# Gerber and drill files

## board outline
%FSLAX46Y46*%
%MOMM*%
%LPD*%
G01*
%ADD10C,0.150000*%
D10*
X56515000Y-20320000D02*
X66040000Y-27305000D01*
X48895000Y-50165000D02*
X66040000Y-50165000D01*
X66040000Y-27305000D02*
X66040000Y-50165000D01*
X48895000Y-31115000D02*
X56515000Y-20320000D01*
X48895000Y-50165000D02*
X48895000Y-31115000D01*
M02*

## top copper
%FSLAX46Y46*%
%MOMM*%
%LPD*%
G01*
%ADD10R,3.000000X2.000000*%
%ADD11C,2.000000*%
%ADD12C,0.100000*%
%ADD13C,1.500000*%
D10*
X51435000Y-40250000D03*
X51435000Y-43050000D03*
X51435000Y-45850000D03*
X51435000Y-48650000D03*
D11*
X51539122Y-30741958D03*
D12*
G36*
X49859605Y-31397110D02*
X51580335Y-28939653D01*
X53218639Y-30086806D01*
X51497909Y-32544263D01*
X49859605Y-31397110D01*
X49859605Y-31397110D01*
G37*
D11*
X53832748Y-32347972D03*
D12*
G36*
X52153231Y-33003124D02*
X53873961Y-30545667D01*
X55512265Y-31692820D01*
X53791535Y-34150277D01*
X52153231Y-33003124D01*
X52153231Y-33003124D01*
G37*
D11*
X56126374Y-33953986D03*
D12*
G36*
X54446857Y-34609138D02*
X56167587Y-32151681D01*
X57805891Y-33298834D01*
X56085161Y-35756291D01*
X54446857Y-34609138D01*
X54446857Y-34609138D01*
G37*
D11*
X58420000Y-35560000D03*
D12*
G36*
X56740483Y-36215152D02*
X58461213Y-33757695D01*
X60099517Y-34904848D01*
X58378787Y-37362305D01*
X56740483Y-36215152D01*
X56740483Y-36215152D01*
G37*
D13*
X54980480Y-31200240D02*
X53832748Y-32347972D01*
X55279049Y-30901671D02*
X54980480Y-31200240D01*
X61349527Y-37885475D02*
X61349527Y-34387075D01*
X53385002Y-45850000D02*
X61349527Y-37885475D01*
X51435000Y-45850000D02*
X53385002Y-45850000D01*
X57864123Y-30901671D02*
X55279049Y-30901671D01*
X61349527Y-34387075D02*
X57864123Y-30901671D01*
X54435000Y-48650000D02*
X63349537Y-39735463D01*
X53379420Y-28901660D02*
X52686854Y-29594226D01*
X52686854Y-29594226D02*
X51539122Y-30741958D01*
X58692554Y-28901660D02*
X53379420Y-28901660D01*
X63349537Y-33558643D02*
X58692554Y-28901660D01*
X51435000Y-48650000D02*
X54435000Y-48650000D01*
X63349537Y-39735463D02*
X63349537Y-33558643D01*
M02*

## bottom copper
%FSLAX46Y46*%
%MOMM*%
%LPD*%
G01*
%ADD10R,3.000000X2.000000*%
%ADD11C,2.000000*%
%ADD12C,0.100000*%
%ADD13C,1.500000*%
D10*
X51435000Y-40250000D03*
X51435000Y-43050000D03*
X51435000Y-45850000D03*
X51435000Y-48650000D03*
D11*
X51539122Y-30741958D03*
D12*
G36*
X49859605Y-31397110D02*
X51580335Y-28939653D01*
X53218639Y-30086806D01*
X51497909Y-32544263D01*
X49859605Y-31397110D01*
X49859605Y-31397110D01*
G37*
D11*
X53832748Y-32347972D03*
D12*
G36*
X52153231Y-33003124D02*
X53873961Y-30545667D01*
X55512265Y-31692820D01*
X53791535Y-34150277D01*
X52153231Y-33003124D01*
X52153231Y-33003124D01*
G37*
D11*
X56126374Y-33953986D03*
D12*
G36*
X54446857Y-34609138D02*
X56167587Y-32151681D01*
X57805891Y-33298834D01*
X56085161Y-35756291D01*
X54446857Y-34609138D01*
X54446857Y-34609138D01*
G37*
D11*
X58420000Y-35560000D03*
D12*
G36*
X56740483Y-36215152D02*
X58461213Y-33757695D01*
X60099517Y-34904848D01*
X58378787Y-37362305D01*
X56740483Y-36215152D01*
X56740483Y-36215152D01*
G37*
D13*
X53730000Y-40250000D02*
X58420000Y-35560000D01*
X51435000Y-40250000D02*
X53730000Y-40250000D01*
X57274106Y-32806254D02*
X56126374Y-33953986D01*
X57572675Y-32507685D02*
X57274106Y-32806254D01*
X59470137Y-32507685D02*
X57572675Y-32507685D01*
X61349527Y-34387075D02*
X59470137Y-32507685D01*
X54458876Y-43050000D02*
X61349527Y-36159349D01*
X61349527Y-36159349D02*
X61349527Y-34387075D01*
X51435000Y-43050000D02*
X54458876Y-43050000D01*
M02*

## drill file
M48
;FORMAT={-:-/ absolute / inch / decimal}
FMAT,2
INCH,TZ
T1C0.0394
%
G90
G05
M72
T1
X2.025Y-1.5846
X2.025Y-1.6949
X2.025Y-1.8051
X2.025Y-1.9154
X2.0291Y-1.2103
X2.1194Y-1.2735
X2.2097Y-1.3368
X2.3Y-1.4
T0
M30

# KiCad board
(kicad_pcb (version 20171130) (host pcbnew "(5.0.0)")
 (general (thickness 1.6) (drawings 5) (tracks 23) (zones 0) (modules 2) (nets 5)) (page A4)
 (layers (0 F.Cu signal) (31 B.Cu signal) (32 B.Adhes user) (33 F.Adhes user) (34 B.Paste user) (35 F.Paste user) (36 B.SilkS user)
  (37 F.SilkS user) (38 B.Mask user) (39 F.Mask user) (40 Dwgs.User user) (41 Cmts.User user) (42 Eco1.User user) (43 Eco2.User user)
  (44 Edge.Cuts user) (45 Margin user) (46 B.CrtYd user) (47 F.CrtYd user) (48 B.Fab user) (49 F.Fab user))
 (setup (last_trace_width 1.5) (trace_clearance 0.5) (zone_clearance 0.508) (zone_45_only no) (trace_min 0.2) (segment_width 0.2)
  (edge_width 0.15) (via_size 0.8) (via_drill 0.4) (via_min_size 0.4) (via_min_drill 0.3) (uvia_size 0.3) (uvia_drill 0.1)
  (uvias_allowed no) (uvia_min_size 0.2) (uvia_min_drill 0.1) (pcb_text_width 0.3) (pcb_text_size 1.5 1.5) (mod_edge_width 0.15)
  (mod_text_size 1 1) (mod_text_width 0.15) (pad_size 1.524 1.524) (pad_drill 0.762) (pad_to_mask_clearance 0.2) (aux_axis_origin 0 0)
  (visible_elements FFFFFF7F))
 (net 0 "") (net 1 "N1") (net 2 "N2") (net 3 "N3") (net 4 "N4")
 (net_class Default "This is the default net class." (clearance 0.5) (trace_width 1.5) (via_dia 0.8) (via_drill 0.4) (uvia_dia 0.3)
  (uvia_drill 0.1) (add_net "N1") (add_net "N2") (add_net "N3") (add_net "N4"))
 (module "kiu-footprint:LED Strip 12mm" (layer F.Cu) (at 51.435 44.45 90)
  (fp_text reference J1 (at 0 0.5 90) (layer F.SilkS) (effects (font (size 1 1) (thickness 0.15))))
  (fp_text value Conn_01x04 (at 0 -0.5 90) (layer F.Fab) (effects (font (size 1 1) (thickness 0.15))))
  (pad 1 thru_hole rect (at 4.2 0 90) (size 2 3) (drill 1) (layers *.Cu *.Mask) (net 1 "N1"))
  (pad 2 thru_hole rect (at 1.4 0 90) (size 2 3) (drill 1) (layers *.Cu *.Mask) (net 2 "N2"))
  (pad 3 thru_hole rect (at -1.4 0 90) (size 2 3) (drill 1) (layers *.Cu *.Mask) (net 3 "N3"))
  (pad 4 thru_hole rect (at -4.2 0 90) (size 2 3) (drill 1) (layers *.Cu *.Mask) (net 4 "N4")))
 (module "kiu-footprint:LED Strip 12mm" (layer F.Cu) (at 54.979561 33.150979 325)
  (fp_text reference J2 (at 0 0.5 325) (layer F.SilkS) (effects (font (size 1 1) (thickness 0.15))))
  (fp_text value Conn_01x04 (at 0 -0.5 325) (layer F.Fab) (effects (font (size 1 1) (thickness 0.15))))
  (pad 4 thru_hole rect (at -4.2 0 325) (size 2 3) (drill 1) (layers *.Cu *.Mask) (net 4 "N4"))
  (pad 3 thru_hole rect (at -1.4 0 325) (size 2 3) (drill 1) (layers *.Cu *.Mask) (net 3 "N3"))
  (pad 2 thru_hole rect (at 1.4 0 325) (size 2 3) (drill 1) (layers *.Cu *.Mask) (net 2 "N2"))
  (pad 1 thru_hole rect (at 4.2 0 325) (size 2 3) (drill 1) (layers *.Cu *.Mask) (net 1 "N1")))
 (gr_line (start 56.515 20.32) (end 66.04 27.305) (layer Edge.Cuts) (width 0.15))
 (gr_line (start 48.895 50.165) (end 66.04 50.165) (layer Edge.Cuts) (width 0.15))
 (gr_line (start 66.04 27.305) (end 66.04 50.165) (layer Edge.Cuts) (width 0.15))
 (gr_line (start 48.895 31.115) (end 56.515 20.32) (layer Edge.Cuts) (width 0.15))
 (gr_line (start 48.895 50.165) (end 48.895 31.115) (layer Edge.Cuts) (width 0.15))
 (segment (start 53.73 40.25) (end 58.42 35.56) (width 1.5) (layer B.Cu) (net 1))
 (segment (start 51.435 40.25) (end 53.73 40.25) (width 1.5) (layer B.Cu) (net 1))
 (segment (start 57.274106 32.806254) (end 56.126374 33.953986) (width 1.5) (layer B.Cu) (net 2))
 (segment (start 57.572675 32.507685) (end 57.274106 32.806254) (width 1.5) (layer B.Cu) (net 2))
 (segment (start 59.470137 32.507685) (end 57.572675 32.507685) (width 1.5) (layer B.Cu) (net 2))
 (segment (start 61.349527 34.387075) (end 59.470137 32.507685) (width 1.5) (layer B.Cu) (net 2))
 (segment (start 54.458876 43.05) (end 61.349527 36.159349) (width 1.5) (layer B.Cu) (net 2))
 (segment (start 61.349527 36.159349) (end 61.349527 34.387075) (width 1.5) (layer B.Cu) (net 2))
 (segment (start 51.435 43.05) (end 54.458876 43.05) (width 1.5) (layer B.Cu) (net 2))
 (segment (start 54.98048 31.20024) (end 53.832748 32.347972) (width 1.5) (layer F.Cu) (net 3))
 (segment (start 55.279049 30.901671) (end 54.98048 31.20024) (width 1.5) (layer F.Cu) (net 3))
 (segment (start 61.349527 37.885475) (end 61.349527 34.387075) (width 1.5) (layer F.Cu) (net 3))
 (segment (start 53.385002 45.85) (end 61.349527 37.885475) (width 1.5) (layer F.Cu) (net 3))
 (segment (start 51.435 45.85) (end 53.385002 45.85) (width 1.5) (layer F.Cu) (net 3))
 (segment (start 57.864123 30.901671) (end 55.279049 30.901671) (width 1.5) (layer F.Cu) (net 3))
 (segment (start 61.349527 34.387075) (end 57.864123 30.901671) (width 1.5) (layer F.Cu) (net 3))
 (segment (start 54.435 48.65) (end 63.349537 39.735463) (width 1.5) (layer F.Cu) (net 4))
 (segment (start 53.37942 28.90166) (end 52.686854 29.594226) (width 1.5) (layer F.Cu) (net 4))
 (segment (start 52.686854 29.594226) (end 51.539122 30.741958) (width 1.5) (layer F.Cu) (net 4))
 (segment (start 58.692554 28.90166) (end 53.37942 28.90166) (width 1.5) (layer F.Cu) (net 4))
 (segment (start 63.349537 33.558643) (end 58.692554 28.90166) (width 1.5) (layer F.Cu) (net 4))
 (segment (start 51.435 48.65) (end 54.435 48.65) (width 1.5) (layer F.Cu) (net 4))
 (segment (start 63.349537 39.735463) (end 63.349537 33.558643) (width 1.5) (layer F.Cu) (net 4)))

